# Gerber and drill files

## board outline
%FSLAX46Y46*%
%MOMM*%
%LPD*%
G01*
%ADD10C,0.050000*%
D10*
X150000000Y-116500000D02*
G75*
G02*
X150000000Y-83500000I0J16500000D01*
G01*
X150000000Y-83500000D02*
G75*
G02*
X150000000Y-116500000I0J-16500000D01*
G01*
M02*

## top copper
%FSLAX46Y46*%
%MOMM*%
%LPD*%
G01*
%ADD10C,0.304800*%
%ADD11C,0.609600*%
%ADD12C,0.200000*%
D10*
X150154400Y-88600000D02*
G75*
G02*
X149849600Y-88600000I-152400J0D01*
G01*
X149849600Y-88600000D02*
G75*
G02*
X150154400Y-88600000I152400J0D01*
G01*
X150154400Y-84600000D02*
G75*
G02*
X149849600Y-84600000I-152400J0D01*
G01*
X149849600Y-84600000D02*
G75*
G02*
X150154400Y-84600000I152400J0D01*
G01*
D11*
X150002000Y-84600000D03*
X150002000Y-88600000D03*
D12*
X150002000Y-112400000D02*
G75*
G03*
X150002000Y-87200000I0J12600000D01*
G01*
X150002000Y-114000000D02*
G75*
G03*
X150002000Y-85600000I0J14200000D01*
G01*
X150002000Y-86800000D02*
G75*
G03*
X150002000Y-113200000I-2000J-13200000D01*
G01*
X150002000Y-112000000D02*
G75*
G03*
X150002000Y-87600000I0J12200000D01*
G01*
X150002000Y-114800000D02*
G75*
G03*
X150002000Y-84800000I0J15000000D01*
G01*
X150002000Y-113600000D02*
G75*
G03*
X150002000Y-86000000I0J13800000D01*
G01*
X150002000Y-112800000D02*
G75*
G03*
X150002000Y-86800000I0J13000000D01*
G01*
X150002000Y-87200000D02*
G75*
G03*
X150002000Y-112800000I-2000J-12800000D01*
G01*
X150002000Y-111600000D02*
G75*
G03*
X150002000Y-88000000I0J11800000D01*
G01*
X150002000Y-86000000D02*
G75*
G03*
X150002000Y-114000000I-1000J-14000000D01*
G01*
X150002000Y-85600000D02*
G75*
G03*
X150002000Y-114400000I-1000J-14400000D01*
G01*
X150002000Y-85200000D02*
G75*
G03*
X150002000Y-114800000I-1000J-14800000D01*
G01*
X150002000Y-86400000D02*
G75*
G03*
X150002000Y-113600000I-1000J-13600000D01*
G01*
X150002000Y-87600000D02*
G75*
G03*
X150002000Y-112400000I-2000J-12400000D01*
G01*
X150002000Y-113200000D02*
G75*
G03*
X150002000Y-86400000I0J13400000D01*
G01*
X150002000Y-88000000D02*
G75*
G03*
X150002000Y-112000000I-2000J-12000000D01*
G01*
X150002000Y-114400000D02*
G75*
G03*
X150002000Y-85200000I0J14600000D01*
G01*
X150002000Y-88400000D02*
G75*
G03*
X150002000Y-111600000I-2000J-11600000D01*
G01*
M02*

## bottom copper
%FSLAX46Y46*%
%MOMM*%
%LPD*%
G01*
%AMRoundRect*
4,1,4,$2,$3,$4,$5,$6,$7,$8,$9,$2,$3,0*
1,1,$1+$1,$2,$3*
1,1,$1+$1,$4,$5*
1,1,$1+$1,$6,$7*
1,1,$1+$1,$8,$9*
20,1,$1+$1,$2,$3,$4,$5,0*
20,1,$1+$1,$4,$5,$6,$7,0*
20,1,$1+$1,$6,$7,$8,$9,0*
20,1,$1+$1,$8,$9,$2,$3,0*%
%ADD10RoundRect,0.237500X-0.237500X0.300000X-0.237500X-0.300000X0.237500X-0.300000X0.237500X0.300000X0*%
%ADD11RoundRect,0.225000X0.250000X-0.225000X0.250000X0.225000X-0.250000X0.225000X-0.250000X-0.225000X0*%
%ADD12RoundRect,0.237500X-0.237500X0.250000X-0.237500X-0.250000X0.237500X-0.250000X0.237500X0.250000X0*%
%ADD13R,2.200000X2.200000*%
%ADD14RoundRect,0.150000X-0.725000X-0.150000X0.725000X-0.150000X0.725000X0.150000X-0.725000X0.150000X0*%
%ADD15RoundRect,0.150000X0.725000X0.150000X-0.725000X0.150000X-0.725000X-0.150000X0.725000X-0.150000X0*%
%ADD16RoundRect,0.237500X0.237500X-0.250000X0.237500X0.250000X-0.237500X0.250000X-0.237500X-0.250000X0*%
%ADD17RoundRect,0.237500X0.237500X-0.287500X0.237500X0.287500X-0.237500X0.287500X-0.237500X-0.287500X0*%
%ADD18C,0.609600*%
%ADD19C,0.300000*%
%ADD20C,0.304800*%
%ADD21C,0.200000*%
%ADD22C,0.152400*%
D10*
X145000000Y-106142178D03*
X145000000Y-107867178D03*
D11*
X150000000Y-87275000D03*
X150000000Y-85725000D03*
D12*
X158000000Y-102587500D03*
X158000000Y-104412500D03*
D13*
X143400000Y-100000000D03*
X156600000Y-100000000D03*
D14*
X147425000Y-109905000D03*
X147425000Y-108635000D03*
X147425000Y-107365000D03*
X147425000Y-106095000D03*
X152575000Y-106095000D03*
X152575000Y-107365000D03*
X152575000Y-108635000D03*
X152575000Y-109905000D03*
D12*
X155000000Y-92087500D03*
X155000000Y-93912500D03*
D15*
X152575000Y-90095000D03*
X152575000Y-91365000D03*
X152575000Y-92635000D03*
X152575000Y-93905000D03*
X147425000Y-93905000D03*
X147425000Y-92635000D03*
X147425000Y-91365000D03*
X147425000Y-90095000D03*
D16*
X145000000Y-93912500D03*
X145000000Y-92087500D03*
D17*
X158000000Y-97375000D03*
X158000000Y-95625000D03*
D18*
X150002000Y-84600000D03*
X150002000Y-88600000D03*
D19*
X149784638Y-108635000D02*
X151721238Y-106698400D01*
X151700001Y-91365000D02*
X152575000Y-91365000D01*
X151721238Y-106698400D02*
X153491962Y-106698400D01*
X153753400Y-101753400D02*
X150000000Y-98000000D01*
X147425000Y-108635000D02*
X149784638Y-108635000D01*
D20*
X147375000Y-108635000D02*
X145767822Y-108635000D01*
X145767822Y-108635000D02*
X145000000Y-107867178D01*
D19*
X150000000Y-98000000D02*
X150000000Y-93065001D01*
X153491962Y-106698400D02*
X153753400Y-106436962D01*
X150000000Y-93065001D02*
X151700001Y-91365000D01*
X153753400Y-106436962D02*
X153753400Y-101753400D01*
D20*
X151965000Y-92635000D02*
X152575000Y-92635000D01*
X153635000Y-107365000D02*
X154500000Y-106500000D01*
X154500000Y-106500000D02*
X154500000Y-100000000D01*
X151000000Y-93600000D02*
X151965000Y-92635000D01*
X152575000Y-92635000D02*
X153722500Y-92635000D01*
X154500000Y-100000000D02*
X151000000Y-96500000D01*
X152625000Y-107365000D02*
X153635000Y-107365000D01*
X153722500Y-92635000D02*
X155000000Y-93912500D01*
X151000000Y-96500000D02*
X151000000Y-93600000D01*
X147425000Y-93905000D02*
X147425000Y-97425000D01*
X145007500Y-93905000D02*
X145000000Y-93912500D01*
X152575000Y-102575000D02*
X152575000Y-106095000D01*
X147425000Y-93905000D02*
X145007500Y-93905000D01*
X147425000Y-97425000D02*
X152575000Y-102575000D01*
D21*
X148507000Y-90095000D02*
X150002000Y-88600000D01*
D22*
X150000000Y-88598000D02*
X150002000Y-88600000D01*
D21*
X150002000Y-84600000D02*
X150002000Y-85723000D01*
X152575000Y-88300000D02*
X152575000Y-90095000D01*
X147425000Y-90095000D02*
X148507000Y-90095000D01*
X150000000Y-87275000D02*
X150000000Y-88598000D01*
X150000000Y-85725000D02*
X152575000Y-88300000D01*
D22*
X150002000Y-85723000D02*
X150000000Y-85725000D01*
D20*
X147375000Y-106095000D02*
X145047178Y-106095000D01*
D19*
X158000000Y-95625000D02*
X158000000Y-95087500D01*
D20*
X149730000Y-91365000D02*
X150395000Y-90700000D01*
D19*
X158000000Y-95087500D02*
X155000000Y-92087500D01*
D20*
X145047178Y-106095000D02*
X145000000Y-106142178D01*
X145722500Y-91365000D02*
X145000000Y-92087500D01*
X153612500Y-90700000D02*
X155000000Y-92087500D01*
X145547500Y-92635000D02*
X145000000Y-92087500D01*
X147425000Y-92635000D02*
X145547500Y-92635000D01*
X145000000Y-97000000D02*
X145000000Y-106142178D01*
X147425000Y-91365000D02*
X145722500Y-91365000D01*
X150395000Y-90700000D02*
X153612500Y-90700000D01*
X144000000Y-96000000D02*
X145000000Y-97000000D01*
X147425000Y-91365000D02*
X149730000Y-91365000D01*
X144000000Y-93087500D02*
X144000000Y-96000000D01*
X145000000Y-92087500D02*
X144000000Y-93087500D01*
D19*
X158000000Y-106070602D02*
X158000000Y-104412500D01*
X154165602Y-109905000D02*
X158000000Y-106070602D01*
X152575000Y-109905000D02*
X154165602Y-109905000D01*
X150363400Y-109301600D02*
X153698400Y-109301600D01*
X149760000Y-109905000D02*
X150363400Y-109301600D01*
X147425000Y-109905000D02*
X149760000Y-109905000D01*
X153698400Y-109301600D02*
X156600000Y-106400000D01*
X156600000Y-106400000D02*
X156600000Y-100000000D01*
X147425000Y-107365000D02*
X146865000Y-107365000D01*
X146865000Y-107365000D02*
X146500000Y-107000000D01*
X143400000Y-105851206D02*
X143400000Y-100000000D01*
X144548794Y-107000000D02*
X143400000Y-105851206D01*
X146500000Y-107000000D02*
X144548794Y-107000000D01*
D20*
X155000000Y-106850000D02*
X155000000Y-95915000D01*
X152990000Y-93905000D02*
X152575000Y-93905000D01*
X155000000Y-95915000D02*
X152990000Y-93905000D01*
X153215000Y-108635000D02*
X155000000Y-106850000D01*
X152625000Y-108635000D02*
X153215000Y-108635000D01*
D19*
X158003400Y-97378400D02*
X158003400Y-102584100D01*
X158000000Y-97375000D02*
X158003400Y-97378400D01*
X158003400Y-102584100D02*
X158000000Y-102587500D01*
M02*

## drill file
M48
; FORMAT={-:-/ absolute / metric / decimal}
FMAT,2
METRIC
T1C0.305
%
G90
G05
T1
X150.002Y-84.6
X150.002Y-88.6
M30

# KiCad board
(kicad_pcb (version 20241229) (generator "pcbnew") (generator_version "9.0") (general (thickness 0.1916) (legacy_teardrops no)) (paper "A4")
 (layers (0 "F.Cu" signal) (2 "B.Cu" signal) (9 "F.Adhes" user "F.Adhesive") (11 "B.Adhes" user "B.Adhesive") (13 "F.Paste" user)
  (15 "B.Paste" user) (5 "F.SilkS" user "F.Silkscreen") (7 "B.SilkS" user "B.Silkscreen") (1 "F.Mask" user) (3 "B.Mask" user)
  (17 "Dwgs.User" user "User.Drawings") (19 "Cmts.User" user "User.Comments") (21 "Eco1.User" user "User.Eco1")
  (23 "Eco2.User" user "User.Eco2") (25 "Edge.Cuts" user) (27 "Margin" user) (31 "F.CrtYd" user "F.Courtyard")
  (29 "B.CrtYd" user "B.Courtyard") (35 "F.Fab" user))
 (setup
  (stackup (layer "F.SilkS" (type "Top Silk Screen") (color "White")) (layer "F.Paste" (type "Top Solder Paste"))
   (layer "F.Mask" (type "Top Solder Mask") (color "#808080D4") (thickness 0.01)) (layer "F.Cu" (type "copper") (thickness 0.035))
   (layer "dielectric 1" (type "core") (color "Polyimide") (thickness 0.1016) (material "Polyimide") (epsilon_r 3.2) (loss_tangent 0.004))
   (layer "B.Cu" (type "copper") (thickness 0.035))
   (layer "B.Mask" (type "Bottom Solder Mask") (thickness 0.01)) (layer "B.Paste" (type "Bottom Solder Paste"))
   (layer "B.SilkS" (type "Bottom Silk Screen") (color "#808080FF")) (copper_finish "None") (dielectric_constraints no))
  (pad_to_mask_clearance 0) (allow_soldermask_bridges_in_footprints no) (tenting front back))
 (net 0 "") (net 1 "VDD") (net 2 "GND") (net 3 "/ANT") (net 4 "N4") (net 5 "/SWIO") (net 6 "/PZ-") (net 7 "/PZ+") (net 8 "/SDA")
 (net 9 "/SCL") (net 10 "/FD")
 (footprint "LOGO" (layer "F.Cu") (at 150 100 -45)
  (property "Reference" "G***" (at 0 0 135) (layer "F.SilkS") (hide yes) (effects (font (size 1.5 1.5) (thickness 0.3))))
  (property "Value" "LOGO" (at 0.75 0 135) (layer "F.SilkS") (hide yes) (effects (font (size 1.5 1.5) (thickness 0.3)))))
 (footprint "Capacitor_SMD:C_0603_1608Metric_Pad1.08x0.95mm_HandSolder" (layer "B.Cu") (at 145 107.004678 -90)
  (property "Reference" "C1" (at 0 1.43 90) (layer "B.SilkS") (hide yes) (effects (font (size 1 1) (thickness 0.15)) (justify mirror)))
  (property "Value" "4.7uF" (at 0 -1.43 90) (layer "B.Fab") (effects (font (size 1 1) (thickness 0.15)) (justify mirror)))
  (pad "1" smd roundrect (at -0.8625 0 270) (size 1.075 0.95) (layers "B.Cu" "B.Mask" "B.Paste") (roundrect_rratio 0.25) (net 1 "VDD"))
  (pad "2" smd roundrect (at 0.8625 0 270) (size 1.075 0.95) (layers "B.Cu" "B.Mask" "B.Paste") (roundrect_rratio 0.25) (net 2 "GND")))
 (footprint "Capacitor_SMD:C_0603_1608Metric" (layer "B.Cu") (at 150 86.5 90)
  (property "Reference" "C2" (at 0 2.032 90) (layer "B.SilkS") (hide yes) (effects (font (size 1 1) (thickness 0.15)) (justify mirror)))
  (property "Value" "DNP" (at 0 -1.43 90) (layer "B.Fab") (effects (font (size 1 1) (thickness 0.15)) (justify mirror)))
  (pad "1" smd roundrect (at -0.775 0 90) (size 0.9 0.95) (layers "B.Cu" "B.Mask" "B.Paste") (roundrect_rratio 0.25) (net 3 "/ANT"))
  (pad "2" smd roundrect (at 0.775 0 90) (size 0.9 0.95) (layers "B.Cu" "B.Mask" "B.Paste") (roundrect_rratio 0.25) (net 3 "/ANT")))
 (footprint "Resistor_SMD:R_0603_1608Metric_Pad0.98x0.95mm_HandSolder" (layer "B.Cu") (at 158 103.5 -90)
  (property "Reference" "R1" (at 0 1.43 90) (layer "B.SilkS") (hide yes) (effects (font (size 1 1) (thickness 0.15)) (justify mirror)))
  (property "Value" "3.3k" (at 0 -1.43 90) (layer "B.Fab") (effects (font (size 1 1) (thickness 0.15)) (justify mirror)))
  (pad "1" smd roundrect (at -0.9125 0 270) (size 0.975 0.95) (layers "B.Cu" "B.Mask" "B.Paste") (roundrect_rratio 0.25) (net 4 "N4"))
  (pad "2" smd roundrect (at 0.9125 0 270) (size 0.975 0.95) (layers "B.Cu" "B.Mask" "B.Paste") (roundrect_rratio 0.25) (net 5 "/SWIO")))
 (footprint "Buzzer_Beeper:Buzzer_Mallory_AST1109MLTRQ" (layer "B.Cu") (at 150 100)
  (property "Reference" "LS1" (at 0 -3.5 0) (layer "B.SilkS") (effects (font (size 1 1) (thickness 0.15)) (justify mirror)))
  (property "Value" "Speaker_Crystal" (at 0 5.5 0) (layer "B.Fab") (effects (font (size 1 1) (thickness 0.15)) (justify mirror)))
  (pad "1" smd rect (at -6.6 0) (size 2.2 2.2) (layers "B.Cu" "B.Mask" "B.Paste") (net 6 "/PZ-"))
  (pad "2" smd rect (at 6.6 0) (size 2.2 2.2) (layers "B.Cu" "B.Mask" "B.Paste") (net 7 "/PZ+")))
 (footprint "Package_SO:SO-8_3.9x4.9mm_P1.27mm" (layer "B.Cu") (at 150 108)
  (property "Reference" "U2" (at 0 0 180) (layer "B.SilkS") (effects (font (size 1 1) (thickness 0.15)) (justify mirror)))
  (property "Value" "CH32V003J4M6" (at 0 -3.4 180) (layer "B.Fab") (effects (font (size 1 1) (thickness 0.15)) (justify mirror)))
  (pad "1" smd roundrect (at -2.575 1.905) (size 1.75 0.6) (layers "B.Cu" "B.Mask" "B.Paste") (roundrect_rratio 0.25) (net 7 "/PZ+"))
  (pad "2" smd roundrect (at -2.575 0.635) (size 1.75 0.6) (layers "B.Cu" "B.Mask" "B.Paste") (roundrect_rratio 0.25) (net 2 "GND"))
  (pad "3" smd roundrect (at -2.575 -0.635) (size 1.75 0.6) (layers "B.Cu" "B.Mask" "B.Paste") (roundrect_rratio 0.25) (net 6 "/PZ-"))
  (pad "4" smd roundrect (at -2.575 -1.905) (size 1.75 0.6) (layers "B.Cu" "B.Mask" "B.Paste") (roundrect_rratio 0.25) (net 1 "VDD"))
  (pad "5" smd roundrect (at 2.575 -1.905) (size 1.75 0.6) (layers "B.Cu" "B.Mask" "B.Paste") (roundrect_rratio 0.25) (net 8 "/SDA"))
  (pad "6" smd roundrect (at 2.575 -0.635) (size 1.75 0.6) (layers "B.Cu" "B.Mask" "B.Paste") (roundrect_rratio 0.25) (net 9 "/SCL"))
  (pad "7" smd roundrect (at 2.575 0.635) (size 1.75 0.6) (layers "B.Cu" "B.Mask" "B.Paste") (roundrect_rratio 0.25) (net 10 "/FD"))
  (pad "8" smd roundrect (at 2.575 1.905) (size 1.75 0.6) (layers "B.Cu" "B.Mask" "B.Paste") (roundrect_rratio 0.25) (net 5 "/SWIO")))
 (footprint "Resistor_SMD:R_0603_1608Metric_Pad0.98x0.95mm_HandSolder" (layer "B.Cu") (at 155 93 -90)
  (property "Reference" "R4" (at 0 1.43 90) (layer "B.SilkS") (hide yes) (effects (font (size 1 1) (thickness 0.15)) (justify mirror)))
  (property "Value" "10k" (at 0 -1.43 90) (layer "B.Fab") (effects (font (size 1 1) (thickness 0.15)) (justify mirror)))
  (pad "1" smd roundrect (at -0.9125 0 270) (size 0.975 0.95) (layers "B.Cu" "B.Mask" "B.Paste") (roundrect_rratio 0.25) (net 1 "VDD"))
  (pad "2" smd roundrect (at 0.9125 0 270) (size 0.975 0.95) (layers "B.Cu" "B.Mask" "B.Paste") (roundrect_rratio 0.25) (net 9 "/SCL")))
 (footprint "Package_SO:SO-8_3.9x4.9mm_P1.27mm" (layer "B.Cu") (at 150 92 180)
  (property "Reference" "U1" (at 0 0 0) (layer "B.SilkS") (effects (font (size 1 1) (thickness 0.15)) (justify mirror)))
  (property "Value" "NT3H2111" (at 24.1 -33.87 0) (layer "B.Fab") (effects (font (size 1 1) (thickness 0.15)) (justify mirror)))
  (pad "1" smd roundrect (at -2.575 1.905 180) (size 1.75 0.6) (layers "B.Cu" "B.Mask" "B.Paste") (roundrect_rratio 0.25) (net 3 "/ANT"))
  (pad "2" smd roundrect (at -2.575 0.635 180) (size 1.75 0.6) (layers "B.Cu" "B.Mask" "B.Paste") (roundrect_rratio 0.25) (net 2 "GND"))
  (pad "3" smd roundrect (at -2.575 -0.635 180) (size 1.75 0.6) (layers "B.Cu" "B.Mask" "B.Paste") (roundrect_rratio 0.25) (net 9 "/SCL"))
  (pad "4" smd roundrect (at -2.575 -1.905 180) (size 1.75 0.6) (layers "B.Cu" "B.Mask" "B.Paste") (roundrect_rratio 0.25) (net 10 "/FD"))
  (pad "5" smd roundrect (at 2.575 -1.905 180) (size 1.75 0.6) (layers "B.Cu" "B.Mask" "B.Paste") (roundrect_rratio 0.25) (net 8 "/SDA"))
  (pad "6" smd roundrect (at 2.575 -0.635 180) (size 1.75 0.6) (layers "B.Cu" "B.Mask" "B.Paste") (roundrect_rratio 0.25) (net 1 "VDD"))
  (pad "7" smd roundrect (at 2.575 0.635 180) (size 1.75 0.6) (layers "B.Cu" "B.Mask" "B.Paste") (roundrect_rratio 0.25) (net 1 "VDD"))
  (pad "8" smd roundrect (at 2.575 1.905 180) (size 1.75 0.6) (layers "B.Cu" "B.Mask" "B.Paste") (roundrect_rratio 0.25) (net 3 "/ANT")))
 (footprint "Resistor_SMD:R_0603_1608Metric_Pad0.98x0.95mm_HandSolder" (layer "B.Cu") (at 145 93 90)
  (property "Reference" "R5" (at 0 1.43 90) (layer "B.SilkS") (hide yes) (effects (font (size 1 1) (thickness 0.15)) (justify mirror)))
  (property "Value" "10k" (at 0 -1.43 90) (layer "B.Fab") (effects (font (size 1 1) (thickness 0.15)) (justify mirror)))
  (pad "1" smd roundrect (at -0.9125 0 90) (size 0.975 0.95) (layers "B.Cu" "B.Mask" "B.Paste") (roundrect_rratio 0.25) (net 8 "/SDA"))
  (pad "2" smd roundrect (at 0.9125 0 90) (size 0.975 0.95) (layers "B.Cu" "B.Mask" "B.Paste") (roundrect_rratio 0.25) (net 1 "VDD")))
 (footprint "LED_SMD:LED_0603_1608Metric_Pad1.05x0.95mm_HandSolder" (layer "B.Cu") (at 158 96.5 90)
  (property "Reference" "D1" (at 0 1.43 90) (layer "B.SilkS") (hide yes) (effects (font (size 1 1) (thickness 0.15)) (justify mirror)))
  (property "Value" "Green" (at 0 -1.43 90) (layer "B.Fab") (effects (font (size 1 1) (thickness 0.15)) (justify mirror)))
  (pad "1" smd roundrect (at -0.875 0 90) (size 1.05 0.95) (layers "B.Cu" "B.Mask" "B.Paste") (roundrect_rratio 0.25) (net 4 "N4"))
  (pad "2" smd roundrect (at 0.875 0 90) (size 1.05 0.95) (layers "B.Cu" "B.Mask" "B.Paste") (roundrect_rratio 0.25) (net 1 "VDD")))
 (gr_circle (center 150.002 88.6) (end 150.3068 88.6) (stroke (width 0) (type solid)) (fill yes) (layer "F.Cu") (net 3))
 (gr_circle (center 150.002 84.6) (end 150.3068 84.6) (stroke (width 0) (type solid)) (fill yes) (layer "F.Cu") (net 3))
 (gr_arc (start 150 116.5) (mid 133.5 100) (end 150 83.5) (stroke (width 0.05) (type solid)) (layer "Edge.Cuts"))
 (gr_arc (start 150 83.5) (mid 166.5 100) (end 150 116.5) (stroke (width 0.05) (type solid)) (layer "Edge.Cuts"))
 (segment (start 149.784638 108.635) (end 151.721238 106.6984) (width 0.3) (layer "B.Cu") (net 2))
 (segment (start 151.700001 91.365) (end 152.575 91.365) (width 0.3) (layer "B.Cu") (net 2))
 (segment (start 151.721238 106.6984) (end 153.491962 106.6984) (width 0.3) (layer "B.Cu") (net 2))
 (segment (start 153.7534 101.7534) (end 150 98) (width 0.3) (layer "B.Cu") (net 2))
 (segment (start 147.425 108.635) (end 149.784638 108.635) (width 0.3) (layer "B.Cu") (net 2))
 (segment (start 147.375 108.635) (end 145.767822 108.635) (width 0.3048) (layer "B.Cu") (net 2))
 (segment (start 145.767822 108.635) (end 145 107.867178) (width 0.3048) (layer "B.Cu") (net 2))
 (segment (start 150 98) (end 150 93.065001) (width 0.3) (layer "B.Cu") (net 2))
 (segment (start 153.491962 106.6984) (end 153.7534 106.436962) (width 0.3) (layer "B.Cu") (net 2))
 (segment (start 150 93.065001) (end 151.700001 91.365) (width 0.3) (layer "B.Cu") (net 2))
 (segment (start 153.7534 106.436962) (end 153.7534 101.7534) (width 0.3) (layer "B.Cu") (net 2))
 (segment (start 151.965 92.635) (end 152.575 92.635) (width 0.3048) (layer "B.Cu") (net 9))
 (segment (start 153.635 107.365) (end 154.5 106.5) (width 0.3048) (layer "B.Cu") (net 9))
 (segment (start 154.5 106.5) (end 154.5 100) (width 0.3048) (layer "B.Cu") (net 9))
 (segment (start 151 93.6) (end 151.965 92.635) (width 0.3048) (layer "B.Cu") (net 9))
 (segment (start 152.575 92.635) (end 153.7225 92.635) (width 0.3048) (layer "B.Cu") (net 9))
 (segment (start 154.5 100) (end 151 96.5) (width 0.3048) (layer "B.Cu") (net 9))
 (segment (start 152.625 107.365) (end 153.635 107.365) (width 0.3048) (layer "B.Cu") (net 9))
 (segment (start 153.7225 92.635) (end 155 93.9125) (width 0.3048) (layer "B.Cu") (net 9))
 (segment (start 151 96.5) (end 151 93.6) (width 0.3048) (layer "B.Cu") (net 9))
 (segment (start 147.425 93.905) (end 147.425 97.425) (width 0.3048) (layer "B.Cu") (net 8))
 (segment (start 145.0075 93.905) (end 145 93.9125) (width 0.3048) (layer "B.Cu") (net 8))
 (segment (start 152.575 102.575) (end 152.575 106.095) (width 0.3048) (layer "B.Cu") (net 8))
 (segment (start 147.425 93.905) (end 145.0075 93.905) (width 0.3048) (layer "B.Cu") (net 8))
 (segment (start 147.425 97.425) (end 152.575 102.575) (width 0.3048) (layer "B.Cu") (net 8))
 (via (at 150.002 84.6) (size 0.6096) (drill 0.3048) (layers "F.Cu" "B.Cu") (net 3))
 (via (at 150.002 88.6) (size 0.6096) (drill 0.3048) (layers "F.Cu" "B.Cu") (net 3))
 (arc (start 150.002 112.4) (mid 162.602 99.8) (end 150.002 87.2) (width 0.2) (layer "F.Cu") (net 3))
 (arc (start 150.002 114) (mid 164.202 99.8) (end 150.002 85.6) (width 0.2) (layer "F.Cu") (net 3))
 (arc (start 150.002 86.8) (mid 136.8 100) (end 150.002 113.2) (width 0.2) (layer "F.Cu") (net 3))
 (arc (start 150.002 112) (mid 162.202 99.8) (end 150.002 87.6) (width 0.2) (layer "F.Cu") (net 3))
 (arc (start 150.002 114.8) (mid 165.002 99.8) (end 150.002 84.8) (width 0.2) (layer "F.Cu") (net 3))
 (arc (start 150.002 113.6) (mid 163.802 99.8) (end 150.002 86) (width 0.2) (layer "F.Cu") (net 3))
 (arc (start 150.002 112.8) (mid 163.002 99.8) (end 150.002 86.8) (width 0.2) (layer "F.Cu") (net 3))
 (arc (start 150.002 87.2) (mid 137.2 100) (end 150.002 112.8) (width 0.2) (layer "F.Cu") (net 3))
 (arc (start 150.002 111.6) (mid 161.802 99.8) (end 150.002 88) (width 0.2) (layer "F.Cu") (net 3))
 (arc (start 150.002 86) (mid 136.001 100) (end 150.002 114) (width 0.2) (layer "F.Cu") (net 3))
 (arc (start 150.002 85.6) (mid 135.601 100) (end 150.002 114.4) (width 0.2) (layer "F.Cu") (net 3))
 (arc (start 150.002 85.2) (mid 135.201 100) (end 150.002 114.8) (width 0.2) (layer "F.Cu") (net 3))
 (arc (start 150.002 86.4) (mid 136.401 100) (end 150.002 113.6) (width 0.2) (layer "F.Cu") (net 3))
 (arc (start 150.002 87.6) (mid 137.6 100) (end 150.002 112.4) (width 0.2) (layer "F.Cu") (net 3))
 (arc (start 150.002 113.2) (mid 163.402 99.8) (end 150.002 86.4) (width 0.2) (layer "F.Cu") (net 3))
 (arc (start 150.002 88) (mid 138 100) (end 150.002 112) (width 0.2) (layer "F.Cu") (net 3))
 (arc (start 150.002 114.4) (mid 164.602 99.8) (end 150.002 85.2) (width 0.2) (layer "F.Cu") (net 3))
 (arc (start 150.002 88.4) (mid 138.4 100) (end 150.002 111.6) (width 0.2) (layer "F.Cu") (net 3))
 (segment (start 148.507 90.095) (end 150.002 88.6) (width 0.2) (layer "B.Cu") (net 3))
 (segment (start 150 88.598) (end 150.002 88.6) (width 0.1524) (layer "B.Cu") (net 3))
 (segment (start 150.002 84.6) (end 150.002 85.723) (width 0.2) (layer "B.Cu") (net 3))
 (segment (start 152.575 88.3) (end 152.575 90.095) (width 0.2) (layer "B.Cu") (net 3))
 (segment (start 147.425 90.095) (end 148.507 90.095) (width 0.2) (layer "B.Cu") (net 3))
 (segment (start 150 87.275) (end 150 88.598) (width 0.2) (layer "B.Cu") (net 3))
 (segment (start 150 85.725) (end 152.575 88.3) (width 0.2) (layer "B.Cu") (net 3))
 (segment (start 150.002 85.723) (end 150 85.725) (width 0.1524) (layer "B.Cu") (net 3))
 (segment (start 147.375 106.095) (end 145.047178 106.095) (width 0.3048) (layer "B.Cu") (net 1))
 (segment (start 158 95.625) (end 158 95.0875) (width 0.3) (layer "B.Cu") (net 1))
 (segment (start 149.73 91.365) (end 150.395 90.7) (width 0.3048) (layer "B.Cu") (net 1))
 (segment (start 158 95.0875) (end 155 92.0875) (width 0.3) (layer "B.Cu") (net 1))
 (segment (start 145.047178 106.095) (end 145 106.142178) (width 0.3048) (layer "B.Cu") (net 1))
 (segment (start 145.7225 91.365) (end 145 92.0875) (width 0.3048) (layer "B.Cu") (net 1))
 (segment (start 153.6125 90.7) (end 155 92.0875) (width 0.3048) (layer "B.Cu") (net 1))
 (segment (start 145.5475 92.635) (end 145 92.0875) (width 0.3048) (layer "B.Cu") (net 1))
 (segment (start 147.425 92.635) (end 145.5475 92.635) (width 0.3048) (layer "B.Cu") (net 1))
 (segment (start 145 97) (end 145 106.142178) (width 0.3048) (layer "B.Cu") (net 1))
 (segment (start 147.425 91.365) (end 145.7225 91.365) (width 0.3048) (layer "B.Cu") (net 1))
 (segment (start 150.395 90.7) (end 153.6125 90.7) (width 0.3048) (layer "B.Cu") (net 1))
 (segment (start 144 96) (end 145 97) (width 0.3048) (layer "B.Cu") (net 1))
 (segment (start 147.425 91.365) (end 149.73 91.365) (width 0.3048) (layer "B.Cu") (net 1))
 (segment (start 144 93.0875) (end 144 96) (width 0.3048) (layer "B.Cu") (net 1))
 (segment (start 145 92.0875) (end 144 93.0875) (width 0.3048) (layer "B.Cu") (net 1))
 (segment (start 158 106.070602) (end 158 104.4125) (width 0.3) (layer "B.Cu") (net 5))
 (segment (start 154.165602 109.905) (end 158 106.070602) (width 0.3) (layer "B.Cu") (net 5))
 (segment (start 152.575 109.905) (end 154.165602 109.905) (width 0.3) (layer "B.Cu") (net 5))
 (segment (start 150.3634 109.3016) (end 153.6984 109.3016) (width 0.3) (layer "B.Cu") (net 7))
 (segment (start 149.76 109.905) (end 150.3634 109.3016) (width 0.3) (layer "B.Cu") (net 7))
 (segment (start 147.425 109.905) (end 149.76 109.905) (width 0.3) (layer "B.Cu") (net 7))
 (segment (start 153.6984 109.3016) (end 156.6 106.4) (width 0.3) (layer "B.Cu") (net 7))
 (segment (start 156.6 106.4) (end 156.6 100) (width 0.3) (layer "B.Cu") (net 7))
 (segment (start 147.425 107.365) (end 146.865 107.365) (width 0.3) (layer "B.Cu") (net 6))
 (segment (start 146.865 107.365) (end 146.5 107) (width 0.3) (layer "B.Cu") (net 6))
 (segment (start 143.4 105.851206) (end 143.4 100) (width 0.3) (layer "B.Cu") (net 6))
 (segment (start 144.548794 107) (end 143.4 105.851206) (width 0.3) (layer "B.Cu") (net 6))
 (segment (start 146.5 107) (end 144.548794 107) (width 0.3) (layer "B.Cu") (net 6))
 (segment (start 155 106.85) (end 155 95.915) (width 0.3048) (layer "B.Cu") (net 10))
 (segment (start 152.99 93.905) (end 152.575 93.905) (width 0.3048) (layer "B.Cu") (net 10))
 (segment (start 155 95.915) (end 152.99 93.905) (width 0.3048) (layer "B.Cu") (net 10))
 (segment (start 153.215 108.635) (end 155 106.85) (width 0.3048) (layer "B.Cu") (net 10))
 (segment (start 152.625 108.635) (end 153.215 108.635) (width 0.3048) (layer "B.Cu") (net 10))
 (segment (start 158.0034 97.3784) (end 158.0034 102.5841) (width 0.3) (layer "B.Cu") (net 4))
 (segment (start 158 97.375) (end 158.0034 97.3784) (width 0.3) (layer "B.Cu") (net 4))
 (segment (start 158.0034 102.5841) (end 158 102.5875) (width 0.3) (layer "B.Cu") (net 4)))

